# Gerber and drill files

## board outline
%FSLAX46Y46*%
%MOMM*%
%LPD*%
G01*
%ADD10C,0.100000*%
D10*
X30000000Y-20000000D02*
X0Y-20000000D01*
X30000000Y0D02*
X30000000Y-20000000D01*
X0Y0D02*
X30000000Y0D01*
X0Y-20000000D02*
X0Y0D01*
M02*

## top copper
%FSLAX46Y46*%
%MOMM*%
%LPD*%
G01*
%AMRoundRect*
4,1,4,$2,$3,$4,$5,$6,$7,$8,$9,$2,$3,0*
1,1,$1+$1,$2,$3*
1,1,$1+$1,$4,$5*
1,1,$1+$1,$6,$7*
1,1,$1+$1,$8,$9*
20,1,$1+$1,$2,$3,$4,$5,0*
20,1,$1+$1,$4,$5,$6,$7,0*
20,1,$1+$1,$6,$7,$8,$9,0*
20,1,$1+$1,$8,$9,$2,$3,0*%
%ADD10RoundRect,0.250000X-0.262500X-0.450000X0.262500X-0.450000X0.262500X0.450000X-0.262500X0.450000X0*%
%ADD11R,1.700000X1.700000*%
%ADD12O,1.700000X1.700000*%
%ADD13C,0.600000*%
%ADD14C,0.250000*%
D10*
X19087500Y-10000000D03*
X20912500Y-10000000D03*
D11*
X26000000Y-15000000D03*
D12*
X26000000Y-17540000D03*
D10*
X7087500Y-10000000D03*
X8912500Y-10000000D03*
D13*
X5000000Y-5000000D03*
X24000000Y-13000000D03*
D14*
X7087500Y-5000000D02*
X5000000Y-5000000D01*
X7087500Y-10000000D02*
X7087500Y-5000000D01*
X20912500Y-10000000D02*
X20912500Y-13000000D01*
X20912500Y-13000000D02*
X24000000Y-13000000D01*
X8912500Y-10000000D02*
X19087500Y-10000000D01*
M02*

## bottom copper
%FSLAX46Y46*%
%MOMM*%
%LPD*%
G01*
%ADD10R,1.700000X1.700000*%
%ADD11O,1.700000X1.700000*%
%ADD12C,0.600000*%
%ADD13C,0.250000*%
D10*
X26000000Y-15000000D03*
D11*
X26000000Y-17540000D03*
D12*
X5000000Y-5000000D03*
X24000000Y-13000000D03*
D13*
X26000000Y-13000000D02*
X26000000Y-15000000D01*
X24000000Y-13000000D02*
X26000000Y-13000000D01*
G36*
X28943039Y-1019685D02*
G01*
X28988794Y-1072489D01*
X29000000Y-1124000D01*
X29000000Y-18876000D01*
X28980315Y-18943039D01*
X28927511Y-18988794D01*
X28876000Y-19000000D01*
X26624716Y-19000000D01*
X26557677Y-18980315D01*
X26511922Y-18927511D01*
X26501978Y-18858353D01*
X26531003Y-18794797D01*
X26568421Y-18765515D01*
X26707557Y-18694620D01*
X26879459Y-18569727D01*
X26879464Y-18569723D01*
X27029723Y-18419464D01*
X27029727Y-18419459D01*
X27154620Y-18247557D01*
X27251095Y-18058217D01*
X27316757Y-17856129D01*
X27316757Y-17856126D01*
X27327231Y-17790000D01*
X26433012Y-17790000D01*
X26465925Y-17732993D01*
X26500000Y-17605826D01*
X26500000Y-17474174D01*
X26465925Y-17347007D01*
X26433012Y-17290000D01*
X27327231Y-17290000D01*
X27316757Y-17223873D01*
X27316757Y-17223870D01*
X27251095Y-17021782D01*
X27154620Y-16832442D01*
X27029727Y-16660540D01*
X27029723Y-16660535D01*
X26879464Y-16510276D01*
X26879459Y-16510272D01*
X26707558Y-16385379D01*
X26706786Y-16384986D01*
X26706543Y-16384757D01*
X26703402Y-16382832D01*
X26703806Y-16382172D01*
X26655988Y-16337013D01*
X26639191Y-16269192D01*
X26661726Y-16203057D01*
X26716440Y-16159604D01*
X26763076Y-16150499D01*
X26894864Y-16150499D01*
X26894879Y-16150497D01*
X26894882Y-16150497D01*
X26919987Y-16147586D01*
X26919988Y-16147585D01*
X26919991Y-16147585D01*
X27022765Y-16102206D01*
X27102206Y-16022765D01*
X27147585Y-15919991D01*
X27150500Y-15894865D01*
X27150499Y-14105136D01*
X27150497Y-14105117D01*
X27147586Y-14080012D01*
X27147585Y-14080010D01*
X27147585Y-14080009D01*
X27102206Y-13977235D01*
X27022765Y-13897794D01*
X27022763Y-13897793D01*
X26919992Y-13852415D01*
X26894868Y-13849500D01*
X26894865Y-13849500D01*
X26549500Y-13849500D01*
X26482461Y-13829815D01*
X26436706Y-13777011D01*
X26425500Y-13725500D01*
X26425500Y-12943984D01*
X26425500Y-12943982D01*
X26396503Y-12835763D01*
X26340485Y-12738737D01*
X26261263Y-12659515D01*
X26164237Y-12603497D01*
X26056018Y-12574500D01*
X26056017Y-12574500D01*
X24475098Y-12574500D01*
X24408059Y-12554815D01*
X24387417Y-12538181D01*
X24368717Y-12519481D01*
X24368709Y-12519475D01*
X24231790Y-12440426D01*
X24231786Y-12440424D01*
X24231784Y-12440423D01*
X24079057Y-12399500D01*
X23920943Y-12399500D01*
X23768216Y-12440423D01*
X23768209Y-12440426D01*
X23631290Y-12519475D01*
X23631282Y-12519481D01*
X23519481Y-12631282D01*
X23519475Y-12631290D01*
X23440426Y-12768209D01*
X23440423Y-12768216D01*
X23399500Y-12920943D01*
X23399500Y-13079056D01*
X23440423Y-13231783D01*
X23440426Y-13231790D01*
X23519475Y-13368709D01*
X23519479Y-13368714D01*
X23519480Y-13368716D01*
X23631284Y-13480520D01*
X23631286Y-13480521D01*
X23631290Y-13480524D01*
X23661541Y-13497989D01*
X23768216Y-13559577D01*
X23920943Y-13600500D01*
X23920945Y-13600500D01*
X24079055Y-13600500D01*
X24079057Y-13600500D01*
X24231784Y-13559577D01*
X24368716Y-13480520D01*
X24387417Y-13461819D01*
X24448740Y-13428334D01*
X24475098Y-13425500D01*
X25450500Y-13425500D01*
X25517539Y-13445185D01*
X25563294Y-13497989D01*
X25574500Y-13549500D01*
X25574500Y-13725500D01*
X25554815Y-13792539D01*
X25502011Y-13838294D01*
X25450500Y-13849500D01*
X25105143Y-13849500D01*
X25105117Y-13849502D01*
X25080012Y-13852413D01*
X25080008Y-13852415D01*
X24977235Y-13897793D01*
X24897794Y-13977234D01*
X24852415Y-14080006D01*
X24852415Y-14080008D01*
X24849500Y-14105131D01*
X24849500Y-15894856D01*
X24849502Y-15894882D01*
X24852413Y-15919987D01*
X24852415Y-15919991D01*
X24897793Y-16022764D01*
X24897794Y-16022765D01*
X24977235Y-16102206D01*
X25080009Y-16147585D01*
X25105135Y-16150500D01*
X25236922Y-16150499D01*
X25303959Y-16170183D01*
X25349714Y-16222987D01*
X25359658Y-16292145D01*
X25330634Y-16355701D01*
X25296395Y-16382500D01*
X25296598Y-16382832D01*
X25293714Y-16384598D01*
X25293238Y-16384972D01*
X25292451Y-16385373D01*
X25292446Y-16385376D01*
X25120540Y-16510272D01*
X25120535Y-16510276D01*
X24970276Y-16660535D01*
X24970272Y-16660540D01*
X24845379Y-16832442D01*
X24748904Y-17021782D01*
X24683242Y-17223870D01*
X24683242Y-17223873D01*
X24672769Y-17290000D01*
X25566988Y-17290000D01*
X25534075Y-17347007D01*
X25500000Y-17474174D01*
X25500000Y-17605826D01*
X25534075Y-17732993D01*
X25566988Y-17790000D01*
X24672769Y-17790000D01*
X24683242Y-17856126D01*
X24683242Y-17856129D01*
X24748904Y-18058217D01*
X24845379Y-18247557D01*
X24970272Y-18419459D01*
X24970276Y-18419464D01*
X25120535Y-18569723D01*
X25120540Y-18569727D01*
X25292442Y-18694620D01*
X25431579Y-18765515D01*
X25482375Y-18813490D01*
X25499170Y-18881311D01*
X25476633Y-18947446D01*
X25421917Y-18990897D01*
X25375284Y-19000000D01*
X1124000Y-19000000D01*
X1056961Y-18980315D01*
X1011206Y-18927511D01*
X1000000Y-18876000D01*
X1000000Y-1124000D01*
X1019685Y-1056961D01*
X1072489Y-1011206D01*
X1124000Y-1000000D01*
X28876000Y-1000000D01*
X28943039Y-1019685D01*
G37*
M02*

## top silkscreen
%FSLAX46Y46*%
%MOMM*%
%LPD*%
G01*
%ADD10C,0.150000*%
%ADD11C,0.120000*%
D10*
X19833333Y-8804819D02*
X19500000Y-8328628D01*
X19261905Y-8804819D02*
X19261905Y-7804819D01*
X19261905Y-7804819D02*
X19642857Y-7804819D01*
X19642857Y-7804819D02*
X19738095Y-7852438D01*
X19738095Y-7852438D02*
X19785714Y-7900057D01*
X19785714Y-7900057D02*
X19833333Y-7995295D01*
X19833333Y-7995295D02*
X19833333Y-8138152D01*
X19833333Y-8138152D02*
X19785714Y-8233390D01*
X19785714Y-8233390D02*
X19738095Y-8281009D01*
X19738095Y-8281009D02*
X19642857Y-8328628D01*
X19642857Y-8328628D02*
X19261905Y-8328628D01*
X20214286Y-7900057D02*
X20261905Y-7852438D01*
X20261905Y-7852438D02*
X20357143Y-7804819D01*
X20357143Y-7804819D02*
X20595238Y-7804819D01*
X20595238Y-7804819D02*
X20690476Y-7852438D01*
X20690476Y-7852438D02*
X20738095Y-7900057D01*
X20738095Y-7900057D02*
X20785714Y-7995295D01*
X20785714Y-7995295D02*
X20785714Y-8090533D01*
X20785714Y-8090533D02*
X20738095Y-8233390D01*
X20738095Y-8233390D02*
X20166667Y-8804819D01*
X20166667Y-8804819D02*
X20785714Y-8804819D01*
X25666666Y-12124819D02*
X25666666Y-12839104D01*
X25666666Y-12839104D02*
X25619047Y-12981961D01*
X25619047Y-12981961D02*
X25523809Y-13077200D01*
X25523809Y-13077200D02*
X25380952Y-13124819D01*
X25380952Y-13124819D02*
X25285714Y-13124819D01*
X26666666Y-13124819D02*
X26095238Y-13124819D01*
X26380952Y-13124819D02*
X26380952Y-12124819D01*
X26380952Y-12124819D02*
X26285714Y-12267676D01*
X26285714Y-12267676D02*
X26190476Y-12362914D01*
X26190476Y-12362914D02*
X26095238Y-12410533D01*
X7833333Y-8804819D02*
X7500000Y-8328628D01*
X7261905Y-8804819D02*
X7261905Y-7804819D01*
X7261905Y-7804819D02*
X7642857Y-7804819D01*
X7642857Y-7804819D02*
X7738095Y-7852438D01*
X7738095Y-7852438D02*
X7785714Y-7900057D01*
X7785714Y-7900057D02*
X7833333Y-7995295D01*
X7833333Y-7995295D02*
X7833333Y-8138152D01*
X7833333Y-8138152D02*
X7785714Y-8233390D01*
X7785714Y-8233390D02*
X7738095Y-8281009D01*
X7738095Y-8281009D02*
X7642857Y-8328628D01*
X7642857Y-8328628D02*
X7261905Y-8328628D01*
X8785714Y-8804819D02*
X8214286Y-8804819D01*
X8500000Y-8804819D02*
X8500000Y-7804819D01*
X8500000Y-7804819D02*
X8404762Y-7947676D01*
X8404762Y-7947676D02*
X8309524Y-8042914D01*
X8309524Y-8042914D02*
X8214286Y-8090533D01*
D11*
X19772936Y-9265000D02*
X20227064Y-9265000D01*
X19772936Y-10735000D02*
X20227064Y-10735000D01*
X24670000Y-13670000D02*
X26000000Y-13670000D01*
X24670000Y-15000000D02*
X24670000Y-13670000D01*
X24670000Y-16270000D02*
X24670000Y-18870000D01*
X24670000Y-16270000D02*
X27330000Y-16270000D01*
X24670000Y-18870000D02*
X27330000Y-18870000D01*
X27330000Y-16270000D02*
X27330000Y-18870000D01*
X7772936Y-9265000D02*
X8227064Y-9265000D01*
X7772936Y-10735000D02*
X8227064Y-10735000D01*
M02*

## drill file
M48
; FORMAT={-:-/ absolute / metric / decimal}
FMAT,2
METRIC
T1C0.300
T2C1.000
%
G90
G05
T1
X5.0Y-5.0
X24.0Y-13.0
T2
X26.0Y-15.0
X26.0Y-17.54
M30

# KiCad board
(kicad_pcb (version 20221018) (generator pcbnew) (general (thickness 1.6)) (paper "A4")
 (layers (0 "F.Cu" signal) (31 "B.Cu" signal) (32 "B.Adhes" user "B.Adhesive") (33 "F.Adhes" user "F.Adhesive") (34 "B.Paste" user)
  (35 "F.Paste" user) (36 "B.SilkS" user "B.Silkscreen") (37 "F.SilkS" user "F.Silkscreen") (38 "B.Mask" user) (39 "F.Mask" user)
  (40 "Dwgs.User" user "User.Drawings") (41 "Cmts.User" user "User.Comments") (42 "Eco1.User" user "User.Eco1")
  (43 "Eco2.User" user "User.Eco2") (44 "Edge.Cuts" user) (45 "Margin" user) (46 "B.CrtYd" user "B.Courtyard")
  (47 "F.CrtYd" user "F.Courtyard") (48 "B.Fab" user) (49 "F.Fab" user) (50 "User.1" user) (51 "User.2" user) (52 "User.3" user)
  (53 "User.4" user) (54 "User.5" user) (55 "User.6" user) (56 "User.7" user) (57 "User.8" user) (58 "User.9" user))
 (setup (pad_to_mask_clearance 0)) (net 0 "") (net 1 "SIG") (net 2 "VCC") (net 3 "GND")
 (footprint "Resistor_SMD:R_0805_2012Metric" (layer "F.Cu") (at 20 10)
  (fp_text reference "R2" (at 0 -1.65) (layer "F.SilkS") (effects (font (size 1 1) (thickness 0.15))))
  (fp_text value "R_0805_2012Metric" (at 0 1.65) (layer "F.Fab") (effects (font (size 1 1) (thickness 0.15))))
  (fp_line (start -0.227064 -0.735) (end 0.227064 -0.735) (stroke (width 0.12) (type solid)) (layer "F.SilkS"))
  (fp_line (start -0.227064 0.735) (end 0.227064 0.735) (stroke (width 0.12) (type solid)) (layer "F.SilkS"))
  (pad "1" smd roundrect (at -0.9125 0) (size 1.025 1.4) (layers "F.Cu" "F.Paste" "F.Mask") (roundrect_rratio 0.243902) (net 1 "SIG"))
  (pad "2" smd roundrect (at 0.9125 0) (size 1.025 1.4) (layers "F.Cu" "F.Paste" "F.Mask") (roundrect_rratio 0.243902) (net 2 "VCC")))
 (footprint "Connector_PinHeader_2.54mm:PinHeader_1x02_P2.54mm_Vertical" (layer "F.Cu") (at 26 15)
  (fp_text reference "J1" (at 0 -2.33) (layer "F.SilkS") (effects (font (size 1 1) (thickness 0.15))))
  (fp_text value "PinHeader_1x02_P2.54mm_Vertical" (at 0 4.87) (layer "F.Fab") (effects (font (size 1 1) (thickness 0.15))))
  (fp_line (start -1.33 -1.33) (end 0 -1.33) (stroke (width 0.12) (type solid)) (layer "F.SilkS"))
  (fp_line (start -1.33 0) (end -1.33 -1.33) (stroke (width 0.12) (type solid)) (layer "F.SilkS"))
  (fp_line (start -1.33 1.27) (end -1.33 3.87) (stroke (width 0.12) (type solid)) (layer "F.SilkS"))
  (fp_line (start -1.33 1.27) (end 1.33 1.27) (stroke (width 0.12) (type solid)) (layer "F.SilkS"))
  (fp_line (start -1.33 3.87) (end 1.33 3.87) (stroke (width 0.12) (type solid)) (layer "F.SilkS"))
  (fp_line (start 1.33 1.27) (end 1.33 3.87) (stroke (width 0.12) (type solid)) (layer "F.SilkS"))
  (pad "1" thru_hole rect (at 0 0) (size 1.7 1.7) (drill 1) (layers "*.Cu" "*.Mask") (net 2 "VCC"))
  (pad "2" thru_hole oval (at 0 2.54) (size 1.7 1.7) (drill 1) (layers "*.Cu" "*.Mask") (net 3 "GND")))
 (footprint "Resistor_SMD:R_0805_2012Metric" (layer "F.Cu") (at 8 10)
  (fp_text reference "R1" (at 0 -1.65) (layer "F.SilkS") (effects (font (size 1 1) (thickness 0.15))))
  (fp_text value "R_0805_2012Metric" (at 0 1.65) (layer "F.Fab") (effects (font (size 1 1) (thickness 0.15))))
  (fp_line (start -0.227064 -0.735) (end 0.227064 -0.735) (stroke (width 0.12) (type solid)) (layer "F.SilkS"))
  (fp_line (start -0.227064 0.735) (end 0.227064 0.735) (stroke (width 0.12) (type solid)) (layer "F.SilkS"))
  (pad "1" smd roundrect (at -0.9125 0) (size 1.025 1.4) (layers "F.Cu" "F.Paste" "F.Mask") (roundrect_rratio 0.243902) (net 3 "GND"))
  (pad "2" smd roundrect (at 0.9125 0) (size 1.025 1.4) (layers "F.Cu" "F.Paste" "F.Mask") (roundrect_rratio 0.243902) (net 1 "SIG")))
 (gr_line (start 30 20) (end 0 20) (stroke (width 0.1) (type default)) (layer "Edge.Cuts"))
 (gr_line (start 30 0) (end 30 20) (stroke (width 0.1) (type default)) (layer "Edge.Cuts"))
 (gr_line (start 0 0) (end 30 0) (stroke (width 0.1) (type default)) (layer "Edge.Cuts"))
 (gr_line (start 0 20) (end 0 0) (stroke (width 0.1) (type default)) (layer "Edge.Cuts"))
 (segment (start 7.0875 5) (end 5 5) (width 0.25) (layer "F.Cu") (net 3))
 (segment (start 7.0875 10) (end 7.0875 5) (width 0.25) (layer "F.Cu") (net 3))
 (via (at 5 5) (size 0.6) (drill 0.3) (layers "F.Cu" "B.Cu") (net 3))
 (segment (start 20.9125 10) (end 20.9125 13) (width 0.25) (layer "F.Cu") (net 2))
 (segment (start 20.9125 13) (end 24 13) (width 0.25) (layer "F.Cu") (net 2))
 (via (at 24 13) (size 0.6) (drill 0.3) (layers "F.Cu" "B.Cu") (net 2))
 (segment (start 26 13) (end 26 15) (width 0.25) (layer "B.Cu") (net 2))
 (segment (start 24 13) (end 26 13) (width 0.25) (layer "B.Cu") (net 2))
 (segment (start 8.9125 10) (end 19.0875 10) (width 0.25) (layer "F.Cu") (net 1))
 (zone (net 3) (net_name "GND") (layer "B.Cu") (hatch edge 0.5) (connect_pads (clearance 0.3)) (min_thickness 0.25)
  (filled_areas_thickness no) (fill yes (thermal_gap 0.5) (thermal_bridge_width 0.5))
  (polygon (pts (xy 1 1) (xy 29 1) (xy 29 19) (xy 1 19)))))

